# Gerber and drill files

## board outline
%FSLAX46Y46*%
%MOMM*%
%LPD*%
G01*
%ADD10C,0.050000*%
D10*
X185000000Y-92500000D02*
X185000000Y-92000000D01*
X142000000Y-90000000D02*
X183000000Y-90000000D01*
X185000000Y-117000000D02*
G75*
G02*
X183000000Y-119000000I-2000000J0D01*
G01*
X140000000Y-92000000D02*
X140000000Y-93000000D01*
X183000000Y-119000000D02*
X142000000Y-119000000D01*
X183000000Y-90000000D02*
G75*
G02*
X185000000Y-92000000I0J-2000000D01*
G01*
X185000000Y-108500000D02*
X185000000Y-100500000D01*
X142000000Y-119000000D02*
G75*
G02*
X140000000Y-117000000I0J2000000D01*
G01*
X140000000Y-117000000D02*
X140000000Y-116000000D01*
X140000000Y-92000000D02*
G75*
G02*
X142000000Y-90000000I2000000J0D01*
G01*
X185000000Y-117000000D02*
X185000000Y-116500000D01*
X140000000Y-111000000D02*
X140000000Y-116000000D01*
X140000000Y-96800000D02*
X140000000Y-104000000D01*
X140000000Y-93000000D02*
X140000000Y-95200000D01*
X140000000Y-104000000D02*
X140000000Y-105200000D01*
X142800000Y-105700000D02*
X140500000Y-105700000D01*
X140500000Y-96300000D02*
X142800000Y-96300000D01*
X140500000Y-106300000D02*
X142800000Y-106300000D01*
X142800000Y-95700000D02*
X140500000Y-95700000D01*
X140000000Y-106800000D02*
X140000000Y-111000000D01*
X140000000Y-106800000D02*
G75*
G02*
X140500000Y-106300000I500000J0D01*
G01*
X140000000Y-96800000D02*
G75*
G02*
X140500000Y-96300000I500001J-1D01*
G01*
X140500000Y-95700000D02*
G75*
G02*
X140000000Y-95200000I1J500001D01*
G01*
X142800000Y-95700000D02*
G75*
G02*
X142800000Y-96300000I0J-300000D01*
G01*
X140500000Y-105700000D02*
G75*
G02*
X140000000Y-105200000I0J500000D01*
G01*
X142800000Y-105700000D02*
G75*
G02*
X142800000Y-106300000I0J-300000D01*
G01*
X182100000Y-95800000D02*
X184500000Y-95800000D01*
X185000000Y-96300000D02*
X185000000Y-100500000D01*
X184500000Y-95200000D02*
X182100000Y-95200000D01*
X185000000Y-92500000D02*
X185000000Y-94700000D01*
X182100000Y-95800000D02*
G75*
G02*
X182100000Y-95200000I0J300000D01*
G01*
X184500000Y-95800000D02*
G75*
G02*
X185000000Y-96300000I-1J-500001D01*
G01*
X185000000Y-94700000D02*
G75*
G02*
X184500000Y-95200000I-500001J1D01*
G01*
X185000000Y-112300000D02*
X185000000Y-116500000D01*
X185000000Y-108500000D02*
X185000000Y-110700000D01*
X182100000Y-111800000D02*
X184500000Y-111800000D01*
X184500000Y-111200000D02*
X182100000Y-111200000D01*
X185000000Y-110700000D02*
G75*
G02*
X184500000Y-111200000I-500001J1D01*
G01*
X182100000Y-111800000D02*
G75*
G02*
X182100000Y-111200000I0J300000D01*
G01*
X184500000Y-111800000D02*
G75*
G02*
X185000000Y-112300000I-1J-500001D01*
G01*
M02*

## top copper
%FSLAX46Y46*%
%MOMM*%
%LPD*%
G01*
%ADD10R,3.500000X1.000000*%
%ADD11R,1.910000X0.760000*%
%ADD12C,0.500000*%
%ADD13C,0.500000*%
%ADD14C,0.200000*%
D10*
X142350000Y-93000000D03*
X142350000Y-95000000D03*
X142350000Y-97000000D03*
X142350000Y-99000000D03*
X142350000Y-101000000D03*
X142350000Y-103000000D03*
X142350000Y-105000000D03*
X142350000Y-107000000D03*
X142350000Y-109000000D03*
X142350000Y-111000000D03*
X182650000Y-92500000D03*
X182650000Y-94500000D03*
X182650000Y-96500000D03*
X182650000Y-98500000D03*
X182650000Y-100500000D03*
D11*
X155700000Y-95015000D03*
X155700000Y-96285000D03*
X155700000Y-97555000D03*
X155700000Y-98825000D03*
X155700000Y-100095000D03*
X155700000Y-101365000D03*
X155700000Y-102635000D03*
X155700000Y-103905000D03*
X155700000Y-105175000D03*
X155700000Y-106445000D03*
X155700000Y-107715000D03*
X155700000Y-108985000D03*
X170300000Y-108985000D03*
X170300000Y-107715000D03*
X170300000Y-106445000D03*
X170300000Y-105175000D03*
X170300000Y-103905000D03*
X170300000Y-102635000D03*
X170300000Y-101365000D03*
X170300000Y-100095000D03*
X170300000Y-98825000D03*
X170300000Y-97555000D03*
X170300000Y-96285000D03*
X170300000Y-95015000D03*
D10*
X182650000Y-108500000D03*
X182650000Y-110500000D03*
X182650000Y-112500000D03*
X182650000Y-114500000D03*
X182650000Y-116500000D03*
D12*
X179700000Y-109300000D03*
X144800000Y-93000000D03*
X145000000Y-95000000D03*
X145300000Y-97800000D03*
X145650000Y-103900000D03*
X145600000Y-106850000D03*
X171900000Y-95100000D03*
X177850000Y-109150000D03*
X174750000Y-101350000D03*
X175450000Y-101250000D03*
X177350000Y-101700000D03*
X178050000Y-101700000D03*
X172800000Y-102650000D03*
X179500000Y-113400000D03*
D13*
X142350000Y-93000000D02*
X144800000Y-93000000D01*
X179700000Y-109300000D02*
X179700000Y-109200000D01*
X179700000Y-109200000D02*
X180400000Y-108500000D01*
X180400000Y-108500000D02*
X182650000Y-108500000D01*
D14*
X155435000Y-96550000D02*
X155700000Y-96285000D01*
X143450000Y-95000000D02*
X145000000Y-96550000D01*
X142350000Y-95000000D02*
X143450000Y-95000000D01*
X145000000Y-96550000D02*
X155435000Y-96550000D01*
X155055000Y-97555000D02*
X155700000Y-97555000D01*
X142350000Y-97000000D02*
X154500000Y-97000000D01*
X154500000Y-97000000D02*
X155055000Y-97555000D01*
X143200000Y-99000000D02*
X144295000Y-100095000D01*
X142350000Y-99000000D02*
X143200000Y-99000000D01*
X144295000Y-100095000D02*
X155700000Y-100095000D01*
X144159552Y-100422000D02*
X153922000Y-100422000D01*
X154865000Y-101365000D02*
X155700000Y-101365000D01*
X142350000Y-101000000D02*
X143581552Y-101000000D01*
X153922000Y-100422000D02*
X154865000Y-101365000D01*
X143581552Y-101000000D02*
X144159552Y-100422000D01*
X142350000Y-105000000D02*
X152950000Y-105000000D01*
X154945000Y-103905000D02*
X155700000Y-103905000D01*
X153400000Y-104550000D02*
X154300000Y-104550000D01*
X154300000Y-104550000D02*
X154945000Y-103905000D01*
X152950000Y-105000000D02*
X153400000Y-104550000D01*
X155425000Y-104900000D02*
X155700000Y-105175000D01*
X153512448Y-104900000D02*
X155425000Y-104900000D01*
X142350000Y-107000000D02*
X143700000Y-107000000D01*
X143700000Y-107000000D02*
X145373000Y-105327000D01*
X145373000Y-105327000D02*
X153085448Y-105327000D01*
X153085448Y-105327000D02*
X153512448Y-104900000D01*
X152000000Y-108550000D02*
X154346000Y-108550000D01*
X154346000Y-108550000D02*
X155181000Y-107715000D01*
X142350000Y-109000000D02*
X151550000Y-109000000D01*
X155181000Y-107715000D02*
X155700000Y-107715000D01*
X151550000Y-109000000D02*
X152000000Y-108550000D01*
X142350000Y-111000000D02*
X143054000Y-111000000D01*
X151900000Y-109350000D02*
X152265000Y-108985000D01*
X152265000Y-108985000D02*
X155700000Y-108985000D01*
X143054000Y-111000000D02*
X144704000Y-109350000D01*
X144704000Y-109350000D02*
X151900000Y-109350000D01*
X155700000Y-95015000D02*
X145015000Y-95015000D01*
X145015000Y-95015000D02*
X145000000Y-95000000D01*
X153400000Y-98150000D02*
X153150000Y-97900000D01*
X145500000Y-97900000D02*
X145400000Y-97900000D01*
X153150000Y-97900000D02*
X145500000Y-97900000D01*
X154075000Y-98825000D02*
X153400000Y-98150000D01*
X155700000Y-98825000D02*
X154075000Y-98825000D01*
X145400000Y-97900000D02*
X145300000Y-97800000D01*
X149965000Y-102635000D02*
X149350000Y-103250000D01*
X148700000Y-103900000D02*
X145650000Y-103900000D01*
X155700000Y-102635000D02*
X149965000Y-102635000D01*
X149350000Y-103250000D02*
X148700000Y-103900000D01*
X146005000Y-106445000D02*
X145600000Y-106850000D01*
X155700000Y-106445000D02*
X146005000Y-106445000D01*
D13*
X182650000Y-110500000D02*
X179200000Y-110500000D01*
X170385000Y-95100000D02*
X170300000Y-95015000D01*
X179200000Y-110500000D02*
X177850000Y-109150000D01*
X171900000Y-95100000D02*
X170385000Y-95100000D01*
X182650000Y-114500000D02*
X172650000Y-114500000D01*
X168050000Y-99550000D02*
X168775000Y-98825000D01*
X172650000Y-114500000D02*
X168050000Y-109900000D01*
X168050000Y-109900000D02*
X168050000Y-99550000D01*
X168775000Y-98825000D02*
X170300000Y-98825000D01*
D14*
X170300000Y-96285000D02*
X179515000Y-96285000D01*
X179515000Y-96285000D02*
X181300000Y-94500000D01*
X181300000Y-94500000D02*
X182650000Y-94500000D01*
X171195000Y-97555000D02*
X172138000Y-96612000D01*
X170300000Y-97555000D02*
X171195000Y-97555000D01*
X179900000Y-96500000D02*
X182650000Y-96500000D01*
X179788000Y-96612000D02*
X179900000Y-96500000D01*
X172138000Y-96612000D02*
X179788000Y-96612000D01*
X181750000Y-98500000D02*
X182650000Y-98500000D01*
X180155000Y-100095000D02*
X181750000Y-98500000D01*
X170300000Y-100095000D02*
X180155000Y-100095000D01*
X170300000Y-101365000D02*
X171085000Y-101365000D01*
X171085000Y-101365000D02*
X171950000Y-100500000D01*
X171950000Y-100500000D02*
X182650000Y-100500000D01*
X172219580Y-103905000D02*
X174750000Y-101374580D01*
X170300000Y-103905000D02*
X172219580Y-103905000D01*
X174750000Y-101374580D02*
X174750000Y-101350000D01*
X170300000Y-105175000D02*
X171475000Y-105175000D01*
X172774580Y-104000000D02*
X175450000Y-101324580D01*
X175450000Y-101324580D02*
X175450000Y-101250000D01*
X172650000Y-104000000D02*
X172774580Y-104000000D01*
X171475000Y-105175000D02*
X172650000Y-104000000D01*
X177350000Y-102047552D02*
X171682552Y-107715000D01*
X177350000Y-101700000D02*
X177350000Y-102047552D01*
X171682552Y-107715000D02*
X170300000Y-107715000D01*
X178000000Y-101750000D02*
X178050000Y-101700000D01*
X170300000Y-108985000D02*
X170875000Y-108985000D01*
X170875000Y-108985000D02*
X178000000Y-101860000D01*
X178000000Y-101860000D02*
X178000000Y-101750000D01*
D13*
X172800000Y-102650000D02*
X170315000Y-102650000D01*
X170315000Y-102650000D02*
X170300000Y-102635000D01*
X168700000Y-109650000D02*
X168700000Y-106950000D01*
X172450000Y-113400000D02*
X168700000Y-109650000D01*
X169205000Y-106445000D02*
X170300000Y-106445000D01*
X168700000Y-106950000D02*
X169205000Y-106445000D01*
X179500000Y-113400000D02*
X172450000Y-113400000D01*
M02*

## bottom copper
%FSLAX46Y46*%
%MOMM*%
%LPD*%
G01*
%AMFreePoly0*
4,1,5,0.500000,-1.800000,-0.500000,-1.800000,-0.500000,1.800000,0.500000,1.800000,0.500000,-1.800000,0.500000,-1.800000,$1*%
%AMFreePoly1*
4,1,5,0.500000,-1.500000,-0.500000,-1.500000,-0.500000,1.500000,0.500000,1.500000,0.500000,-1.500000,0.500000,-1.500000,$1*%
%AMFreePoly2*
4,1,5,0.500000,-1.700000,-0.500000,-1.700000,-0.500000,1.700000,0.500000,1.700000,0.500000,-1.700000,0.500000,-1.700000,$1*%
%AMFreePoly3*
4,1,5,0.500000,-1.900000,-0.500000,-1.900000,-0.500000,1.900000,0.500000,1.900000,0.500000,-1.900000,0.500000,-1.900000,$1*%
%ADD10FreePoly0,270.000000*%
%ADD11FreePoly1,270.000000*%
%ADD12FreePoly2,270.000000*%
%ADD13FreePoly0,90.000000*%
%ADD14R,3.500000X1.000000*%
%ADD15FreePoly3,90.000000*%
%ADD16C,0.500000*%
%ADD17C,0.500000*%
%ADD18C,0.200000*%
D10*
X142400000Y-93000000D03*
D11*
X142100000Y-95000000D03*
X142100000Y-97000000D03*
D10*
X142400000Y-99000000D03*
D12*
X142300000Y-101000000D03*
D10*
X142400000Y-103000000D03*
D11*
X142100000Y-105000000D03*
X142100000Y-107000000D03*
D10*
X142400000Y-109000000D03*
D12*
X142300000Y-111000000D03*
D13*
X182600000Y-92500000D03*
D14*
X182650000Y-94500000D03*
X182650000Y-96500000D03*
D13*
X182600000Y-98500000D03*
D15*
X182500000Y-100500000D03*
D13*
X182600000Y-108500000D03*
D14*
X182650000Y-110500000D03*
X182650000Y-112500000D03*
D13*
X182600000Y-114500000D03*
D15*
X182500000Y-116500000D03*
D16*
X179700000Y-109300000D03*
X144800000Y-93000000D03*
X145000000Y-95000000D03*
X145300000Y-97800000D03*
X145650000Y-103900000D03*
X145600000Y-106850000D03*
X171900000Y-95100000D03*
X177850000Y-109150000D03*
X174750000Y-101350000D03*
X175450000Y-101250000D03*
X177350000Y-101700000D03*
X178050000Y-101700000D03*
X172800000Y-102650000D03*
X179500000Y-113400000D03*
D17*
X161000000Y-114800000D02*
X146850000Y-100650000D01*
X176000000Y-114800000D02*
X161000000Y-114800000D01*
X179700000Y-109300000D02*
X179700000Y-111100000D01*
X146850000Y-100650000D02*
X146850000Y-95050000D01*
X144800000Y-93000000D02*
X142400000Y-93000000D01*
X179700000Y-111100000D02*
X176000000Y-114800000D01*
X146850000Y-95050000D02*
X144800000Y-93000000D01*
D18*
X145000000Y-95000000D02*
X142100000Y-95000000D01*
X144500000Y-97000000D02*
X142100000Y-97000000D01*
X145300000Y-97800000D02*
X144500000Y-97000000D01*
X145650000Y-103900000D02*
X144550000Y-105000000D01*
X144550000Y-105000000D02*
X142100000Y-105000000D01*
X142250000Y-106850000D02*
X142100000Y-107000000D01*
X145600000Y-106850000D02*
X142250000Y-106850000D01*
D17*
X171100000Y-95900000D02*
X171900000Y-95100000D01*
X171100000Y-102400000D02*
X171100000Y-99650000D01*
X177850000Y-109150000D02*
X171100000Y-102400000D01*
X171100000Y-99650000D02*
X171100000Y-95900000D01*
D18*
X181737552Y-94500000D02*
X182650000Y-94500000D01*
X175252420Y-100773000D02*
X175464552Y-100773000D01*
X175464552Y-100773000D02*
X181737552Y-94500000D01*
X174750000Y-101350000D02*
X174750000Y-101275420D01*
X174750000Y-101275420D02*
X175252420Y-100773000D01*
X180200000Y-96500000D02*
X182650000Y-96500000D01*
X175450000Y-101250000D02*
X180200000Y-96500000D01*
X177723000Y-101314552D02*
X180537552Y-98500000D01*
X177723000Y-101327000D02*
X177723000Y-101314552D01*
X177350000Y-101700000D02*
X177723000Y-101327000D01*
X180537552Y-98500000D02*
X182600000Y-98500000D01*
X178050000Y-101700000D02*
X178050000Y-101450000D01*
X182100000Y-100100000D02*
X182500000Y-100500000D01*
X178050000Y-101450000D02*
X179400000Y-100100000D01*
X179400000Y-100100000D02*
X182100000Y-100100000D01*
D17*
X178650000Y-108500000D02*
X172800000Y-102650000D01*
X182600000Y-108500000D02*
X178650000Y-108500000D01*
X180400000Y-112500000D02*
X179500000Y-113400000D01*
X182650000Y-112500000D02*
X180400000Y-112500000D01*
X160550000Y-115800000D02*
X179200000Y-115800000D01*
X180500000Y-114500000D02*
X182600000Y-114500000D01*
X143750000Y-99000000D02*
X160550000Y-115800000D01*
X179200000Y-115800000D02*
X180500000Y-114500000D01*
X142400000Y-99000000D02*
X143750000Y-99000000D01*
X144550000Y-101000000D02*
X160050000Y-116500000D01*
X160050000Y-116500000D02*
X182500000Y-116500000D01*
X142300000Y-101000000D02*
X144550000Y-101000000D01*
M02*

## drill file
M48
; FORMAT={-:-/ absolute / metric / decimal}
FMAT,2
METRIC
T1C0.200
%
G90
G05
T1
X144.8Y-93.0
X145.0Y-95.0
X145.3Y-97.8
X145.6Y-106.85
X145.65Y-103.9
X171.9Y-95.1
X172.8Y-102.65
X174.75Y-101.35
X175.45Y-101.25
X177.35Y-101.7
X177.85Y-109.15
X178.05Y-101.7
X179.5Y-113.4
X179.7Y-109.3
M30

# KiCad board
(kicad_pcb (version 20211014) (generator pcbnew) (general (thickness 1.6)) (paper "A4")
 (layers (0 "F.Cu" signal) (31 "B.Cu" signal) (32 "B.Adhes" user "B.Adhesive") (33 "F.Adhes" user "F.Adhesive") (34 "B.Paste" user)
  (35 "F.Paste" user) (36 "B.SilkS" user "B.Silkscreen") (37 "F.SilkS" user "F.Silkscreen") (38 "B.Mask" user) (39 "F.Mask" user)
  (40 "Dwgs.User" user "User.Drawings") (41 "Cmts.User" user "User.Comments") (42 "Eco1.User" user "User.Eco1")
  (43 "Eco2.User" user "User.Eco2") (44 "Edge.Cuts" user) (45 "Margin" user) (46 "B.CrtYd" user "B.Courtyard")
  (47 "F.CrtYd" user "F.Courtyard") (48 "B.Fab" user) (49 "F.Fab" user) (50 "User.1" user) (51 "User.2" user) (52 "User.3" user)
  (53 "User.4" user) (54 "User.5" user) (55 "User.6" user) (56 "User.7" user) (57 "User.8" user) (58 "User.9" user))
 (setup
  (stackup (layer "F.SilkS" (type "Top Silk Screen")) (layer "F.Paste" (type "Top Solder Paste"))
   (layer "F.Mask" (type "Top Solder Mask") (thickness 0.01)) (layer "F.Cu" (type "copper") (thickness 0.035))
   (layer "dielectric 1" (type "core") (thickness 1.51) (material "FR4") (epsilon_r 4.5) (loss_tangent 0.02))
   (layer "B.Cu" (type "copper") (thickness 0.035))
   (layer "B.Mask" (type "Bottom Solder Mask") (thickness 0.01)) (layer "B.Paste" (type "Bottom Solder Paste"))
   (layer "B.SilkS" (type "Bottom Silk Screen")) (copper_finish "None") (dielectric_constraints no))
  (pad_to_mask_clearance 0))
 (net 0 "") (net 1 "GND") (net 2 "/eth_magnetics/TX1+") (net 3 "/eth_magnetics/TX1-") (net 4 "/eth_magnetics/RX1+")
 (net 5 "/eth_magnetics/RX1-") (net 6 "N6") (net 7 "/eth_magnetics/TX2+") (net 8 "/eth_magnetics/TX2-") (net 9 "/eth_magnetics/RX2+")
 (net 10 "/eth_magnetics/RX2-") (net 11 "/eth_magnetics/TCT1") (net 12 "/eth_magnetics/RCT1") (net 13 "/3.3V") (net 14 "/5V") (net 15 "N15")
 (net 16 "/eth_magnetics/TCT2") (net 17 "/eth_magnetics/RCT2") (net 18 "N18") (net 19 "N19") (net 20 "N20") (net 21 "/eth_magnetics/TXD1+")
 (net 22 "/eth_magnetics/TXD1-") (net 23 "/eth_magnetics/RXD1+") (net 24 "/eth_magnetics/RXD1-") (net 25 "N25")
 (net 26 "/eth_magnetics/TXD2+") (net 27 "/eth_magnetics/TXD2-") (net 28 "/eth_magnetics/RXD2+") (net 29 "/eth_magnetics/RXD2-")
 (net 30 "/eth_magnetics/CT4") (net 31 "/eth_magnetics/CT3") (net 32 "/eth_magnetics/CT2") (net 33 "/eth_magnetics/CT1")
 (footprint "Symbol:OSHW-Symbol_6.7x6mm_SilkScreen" (layer "F.Cu") (at 158 116)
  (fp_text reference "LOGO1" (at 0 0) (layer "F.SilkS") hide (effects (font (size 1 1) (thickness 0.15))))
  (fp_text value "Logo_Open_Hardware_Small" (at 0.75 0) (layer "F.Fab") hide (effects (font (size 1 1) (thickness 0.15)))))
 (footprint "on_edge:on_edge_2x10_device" (layer "F.Cu") (at 140 97 -90)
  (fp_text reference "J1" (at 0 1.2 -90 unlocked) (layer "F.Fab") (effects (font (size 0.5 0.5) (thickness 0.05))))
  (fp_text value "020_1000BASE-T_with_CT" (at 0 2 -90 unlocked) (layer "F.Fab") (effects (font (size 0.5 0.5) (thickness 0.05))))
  (fp_line (start -0.2 0) (end 7 0) (layer "Edge.Cuts") (width 0.05))
  (fp_line (start -4 0) (end -1.8 0) (layer "Edge.Cuts") (width 0.05))
  (fp_line (start 7 0) (end 8.2 0) (layer "Edge.Cuts") (width 0.05))
  (fp_line (start 8.7 -2.8) (end 8.7 -0.5) (layer "Edge.Cuts") (width 0.05))
  (fp_line (start -0.7 -0.5) (end -0.7 -2.8) (layer "Edge.Cuts") (width 0.05))
  (fp_line (start 9.3 -0.5) (end 9.3 -2.8) (layer "Edge.Cuts") (width 0.05))
  (fp_line (start -1.3 -2.8) (end -1.3 -0.5) (layer "Edge.Cuts") (width 0.05))
  (fp_line (start 9.8 0) (end 14 0) (layer "Edge.Cuts") (width 0.05))
  (fp_arc (start 9.8 0) (mid 9.446447 -0.146447) (end 9.3 -0.5) (layer "Edge.Cuts") (width 0.05))
  (fp_arc (start -0.2 0) (mid -0.553553 -0.146447) (end -0.7 -0.5) (layer "Edge.Cuts") (width 0.05))
  (fp_arc (start -1.3 -0.5) (mid -1.446447 -0.146447) (end -1.8 0) (layer "Edge.Cuts") (width 0.05))
  (fp_arc (start -1.3 -2.8) (mid -1 -3.1) (end -0.7 -2.8) (layer "Edge.Cuts") (width 0.05))
  (fp_arc (start 8.7 -0.5) (mid 8.553553 -0.146447) (end 8.2 0) (layer "Edge.Cuts") (width 0.05))
  (fp_arc (start 8.7 -2.8) (mid 9 -3.1) (end 9.3 -2.8) (layer "Edge.Cuts") (width 0.05))
  (pad "1" smd rect (at -4 -2.35 90) (size 1 3.5) (layers "F.Cu" "F.Mask") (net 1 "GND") (zone_connect 0))
  (pad "2" smd rect (at -2 -2.35 270) (size 1 3.5) (layers "F.Cu" "F.Mask") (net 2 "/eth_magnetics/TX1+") (zone_connect 0))
  (pad "3" smd rect (at 0 -2.35 270) (size 1 3.5) (layers "F.Cu" "F.Mask") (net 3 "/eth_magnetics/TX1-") (zone_connect 0))
  (pad "4" smd rect (at 2 -2.35 90) (size 1 3.5) (layers "F.Cu" "F.Mask") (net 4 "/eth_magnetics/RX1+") (zone_connect 0))
  (pad "5" smd rect (at 4 -2.35 90) (size 1 3.5) (layers "F.Cu" "F.Mask") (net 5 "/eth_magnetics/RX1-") (zone_connect 0))
  (pad "6" smd rect (at 6 -2.35 90) (size 1 3.5) (layers "F.Cu" "F.Mask") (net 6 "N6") (zone_connect 0))
  (pad "7" smd rect (at 8 -2.35 270) (size 1 3.5) (layers "F.Cu" "F.Mask") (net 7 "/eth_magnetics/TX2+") (zone_connect 0))
  (pad "8" smd rect (at 10 -2.35 270) (size 1 3.5) (layers "F.Cu" "F.Mask") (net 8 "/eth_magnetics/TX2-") (zone_connect 0))
  (pad "9" smd rect (at 12 -2.35 90) (size 1 3.5) (layers "F.Cu" "F.Mask") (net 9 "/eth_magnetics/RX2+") (zone_connect 0))
  (pad "10" smd rect (at 14 -2.35 90) (size 1 3.5) (layers "F.Cu" "F.Mask") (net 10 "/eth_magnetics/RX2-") (zone_connect 0))
  (pad "11" smd custom (at -4 -2.4 270) (size 1 3.6) (layers "B.Cu" "B.Mask") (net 1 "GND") (zone_connect 0)
   (options (clearance outline) (anchor rect)) (primitives))
  (pad "12" smd custom (at -2 -2.1 270) (size 1 3) (layers "B.Cu" "B.Mask") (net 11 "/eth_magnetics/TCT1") (zone_connect 0)
   (options (clearance outline) (anchor rect)) (primitives))
  (pad "13" smd custom (at 0 -2.1 270) (size 1 3) (layers "B.Cu" "B.Mask") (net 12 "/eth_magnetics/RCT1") (zone_connect 0)
   (options (clearance outline) (anchor rect)) (primitives))
  (pad "14" smd custom (at 2 -2.4 270) (size 1 3.6) (layers "B.Cu" "B.Mask") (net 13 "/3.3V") (zone_connect 0)
   (options (clearance outline) (anchor rect)) (primitives))
  (pad "15" smd custom (at 4 -2.3 270) (size 1 3.4) (layers "B.Cu" "B.Mask") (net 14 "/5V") (zone_connect 0)
   (options (clearance outline) (anchor rect)) (primitives))
  (pad "16" smd custom (at 6 -2.4 270) (size 1 3.6) (layers "B.Cu" "B.Mask") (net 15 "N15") (zone_connect 0)
   (options (clearance outline) (anchor rect)) (primitives))
  (pad "17" smd custom (at 8 -2.1 270) (size 1 3) (layers "B.Cu" "B.Mask") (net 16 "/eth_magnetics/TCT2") (zone_connect 0)
   (options (clearance outline) (anchor rect)) (primitives))
  (pad "18" smd custom (at 10 -2.1 270) (size 1 3) (layers "B.Cu" "B.Mask") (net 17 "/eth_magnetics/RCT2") (zone_connect 0)
   (options (clearance outline) (anchor rect)) (primitives))
  (pad "19" smd custom (at 12 -2.4 270) (size 1 3.6) (layers "B.Cu" "B.Mask") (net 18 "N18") (zone_connect 0)
   (options (clearance outline) (anchor rect)) (primitives))
  (pad "20" smd custom (at 14 -2.3 270) (size 1 3.4) (layers "B.Cu" "B.Mask") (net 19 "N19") (zone_connect 0)
   (options (clearance outline) (anchor rect)) (primitives))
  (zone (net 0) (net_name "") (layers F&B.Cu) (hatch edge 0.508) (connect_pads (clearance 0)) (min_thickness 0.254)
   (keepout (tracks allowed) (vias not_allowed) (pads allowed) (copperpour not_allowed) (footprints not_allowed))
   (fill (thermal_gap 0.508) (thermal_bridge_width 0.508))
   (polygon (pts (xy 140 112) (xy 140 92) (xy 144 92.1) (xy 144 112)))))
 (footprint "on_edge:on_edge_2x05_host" (layer "F.Cu") (at 185 96.5 -90)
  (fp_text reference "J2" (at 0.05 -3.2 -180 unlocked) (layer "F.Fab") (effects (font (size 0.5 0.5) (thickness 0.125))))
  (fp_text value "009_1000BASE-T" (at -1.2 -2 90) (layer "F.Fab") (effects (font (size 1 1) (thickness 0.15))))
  (fp_line (start -0.7 2.9) (end -0.7 0.5) (layer "Edge.Cuts") (width 0.05))
  (fp_line (start -0.2 0) (end 4 0) (layer "Edge.Cuts") (width 0.05))
  (fp_line (start -1.3 0.5) (end -1.3 2.9) (layer "Edge.Cuts") (width 0.05))
  (fp_line (start -4 0) (end -1.8 0) (layer "Edge.Cuts") (width 0.05))
  (fp_arc (start -0.7 2.9) (mid -1 3.2) (end -1.3 2.9) (layer "Edge.Cuts") (width 0.05))
  (fp_arc (start -0.7 0.5) (mid -0.553553 0.146447) (end -0.2 0) (layer "Edge.Cuts") (width 0.05))
  (fp_arc (start -1.8 0) (mid -1.446447 0.146447) (end -1.3 0.5) (layer "Edge.Cuts") (width 0.05))
  (pad "1" smd rect (at -4 2.35 270) (size 1 3.5) (layers "F.Cu" "F.Mask") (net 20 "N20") (zone_connect 0))
  (pad "2" smd rect (at -2 2.35 270) (size 1 3.5) (layers "F.Cu" "F.Mask") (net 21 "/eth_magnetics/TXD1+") (zone_connect 0))
  (pad "3" smd rect (at 0 2.35 270) (size 1 3.5) (layers "F.Cu" "F.Mask") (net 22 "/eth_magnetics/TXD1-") (zone_connect 0))
  (pad "4" smd rect (at 2 2.35 270) (size 1 3.5) (layers "F.Cu" "F.Mask") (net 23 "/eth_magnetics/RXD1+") (zone_connect 0))
  (pad "5" smd rect (at 4 2.35 270) (size 1 3.5) (layers "F.Cu" "F.Mask") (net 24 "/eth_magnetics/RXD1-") (zone_connect 0))
  (pad "6" smd custom (at -4 2.4 90) (size 1 3.6) (layers "B.Cu" "B.Mask") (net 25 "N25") (zone_connect 0)
   (options (clearance outline) (anchor rect)) (primitives))
  (pad "7" smd rect (at -2 2.35 90) (size 1 3.5) (layers "B.Cu" "B.Mask") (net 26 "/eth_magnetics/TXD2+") (zone_connect 0))
  (pad "8" smd rect (at 0 2.35 90) (size 1 3.5) (layers "B.Cu" "B.Mask") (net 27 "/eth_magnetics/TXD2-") (zone_connect 0))
  (pad "9" smd custom (at 2 2.4 90) (size 1 3.6) (layers "B.Cu" "B.Mask") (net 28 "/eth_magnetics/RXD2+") (zone_connect 0)
   (options (clearance outline) (anchor rect)) (primitives))
  (pad "10" smd custom (at 4 2.5 90) (size 1 3.8) (layers "B.Cu" "B.Mask") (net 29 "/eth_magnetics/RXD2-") (zone_connect 0)
   (options (clearance outline) (anchor rect)) (primitives))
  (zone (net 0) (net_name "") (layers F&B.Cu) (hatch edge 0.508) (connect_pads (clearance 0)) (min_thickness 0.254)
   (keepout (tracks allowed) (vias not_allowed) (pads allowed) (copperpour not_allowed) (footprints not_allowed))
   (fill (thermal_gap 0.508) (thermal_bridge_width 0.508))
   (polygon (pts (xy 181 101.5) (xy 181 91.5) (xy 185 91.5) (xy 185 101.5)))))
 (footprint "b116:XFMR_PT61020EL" (layer "F.Cu") (at 163 102)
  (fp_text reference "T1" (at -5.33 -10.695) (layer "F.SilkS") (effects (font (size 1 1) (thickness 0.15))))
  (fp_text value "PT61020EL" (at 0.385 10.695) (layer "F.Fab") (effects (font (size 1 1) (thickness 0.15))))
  (pad "1" smd rect (at -7.3 -6.985) (size 1.91 0.76) (layers "F.Cu" "F.Paste" "F.Mask") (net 11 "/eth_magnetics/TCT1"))
  (pad "2" smd rect (at -7.3 -5.715) (size 1.91 0.76) (layers "F.Cu" "F.Paste" "F.Mask") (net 2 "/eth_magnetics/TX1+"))
  (pad "3" smd rect (at -7.3 -4.445) (size 1.91 0.76) (layers "F.Cu" "F.Paste" "F.Mask") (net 3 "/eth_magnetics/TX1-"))
  (pad "4" smd rect (at -7.3 -3.175) (size 1.91 0.76) (layers "F.Cu" "F.Paste" "F.Mask") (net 12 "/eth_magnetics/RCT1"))
  (pad "5" smd rect (at -7.3 -1.905) (size 1.91 0.76) (layers "F.Cu" "F.Paste" "F.Mask") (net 4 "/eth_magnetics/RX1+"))
  (pad "6" smd rect (at -7.3 -0.635) (size 1.91 0.76) (layers "F.Cu" "F.Paste" "F.Mask") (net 5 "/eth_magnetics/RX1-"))
  (pad "7" smd rect (at -7.3 0.635) (size 1.91 0.76) (layers "F.Cu" "F.Paste" "F.Mask") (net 16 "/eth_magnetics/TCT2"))
  (pad "8" smd rect (at -7.3 1.905) (size 1.91 0.76) (layers "F.Cu" "F.Paste" "F.Mask") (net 7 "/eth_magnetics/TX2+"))
  (pad "9" smd rect (at -7.3 3.175) (size 1.91 0.76) (layers "F.Cu" "F.Paste" "F.Mask") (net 8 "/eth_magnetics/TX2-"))
  (pad "10" smd rect (at -7.3 4.445) (size 1.91 0.76) (layers "F.Cu" "F.Paste" "F.Mask") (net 17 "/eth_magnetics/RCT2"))
  (pad "11" smd rect (at -7.3 5.715) (size 1.91 0.76) (layers "F.Cu" "F.Paste" "F.Mask") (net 9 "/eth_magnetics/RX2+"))
  (pad "12" smd rect (at -7.3 6.985) (size 1.91 0.76) (layers "F.Cu" "F.Paste" "F.Mask") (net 10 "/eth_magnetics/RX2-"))
  (pad "13" smd rect (at 7.3 6.985) (size 1.91 0.76) (layers "F.Cu" "F.Paste" "F.Mask") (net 29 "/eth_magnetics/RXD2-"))
  (pad "14" smd rect (at 7.3 5.715) (size 1.91 0.76) (layers "F.Cu" "F.Paste" "F.Mask") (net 28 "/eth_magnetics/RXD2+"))
  (pad "15" smd rect (at 7.3 4.445) (size 1.91 0.76) (layers "F.Cu" "F.Paste" "F.Mask") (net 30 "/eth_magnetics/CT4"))
  (pad "16" smd rect (at 7.3 3.175) (size 1.91 0.76) (layers "F.Cu" "F.Paste" "F.Mask") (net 27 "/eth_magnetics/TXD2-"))
  (pad "17" smd rect (at 7.3 1.905) (size 1.91 0.76) (layers "F.Cu" "F.Paste" "F.Mask") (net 26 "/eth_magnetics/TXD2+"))
  (pad "18" smd rect (at 7.3 0.635) (size 1.91 0.76) (layers "F.Cu" "F.Paste" "F.Mask") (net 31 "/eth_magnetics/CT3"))
  (pad "19" smd rect (at 7.3 -0.635) (size 1.91 0.76) (layers "F.Cu" "F.Paste" "F.Mask") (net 24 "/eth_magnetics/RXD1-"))
  (pad "20" smd rect (at 7.3 -1.905) (size 1.91 0.76) (layers "F.Cu" "F.Paste" "F.Mask") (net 23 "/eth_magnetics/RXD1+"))
  (pad "21" smd rect (at 7.3 -3.175) (size 1.91 0.76) (layers "F.Cu" "F.Paste" "F.Mask") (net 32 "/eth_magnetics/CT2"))
  (pad "22" smd rect (at 7.3 -4.445) (size 1.91 0.76) (layers "F.Cu" "F.Paste" "F.Mask") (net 22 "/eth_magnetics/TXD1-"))
  (pad "23" smd rect (at 7.3 -5.715) (size 1.91 0.76) (layers "F.Cu" "F.Paste" "F.Mask") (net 21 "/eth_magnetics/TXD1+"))
  (pad "24" smd rect (at 7.3 -6.985) (size 1.91 0.76) (layers "F.Cu" "F.Paste" "F.Mask") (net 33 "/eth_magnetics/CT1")))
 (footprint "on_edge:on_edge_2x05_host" (layer "F.Cu") (at 185 112.5 -90)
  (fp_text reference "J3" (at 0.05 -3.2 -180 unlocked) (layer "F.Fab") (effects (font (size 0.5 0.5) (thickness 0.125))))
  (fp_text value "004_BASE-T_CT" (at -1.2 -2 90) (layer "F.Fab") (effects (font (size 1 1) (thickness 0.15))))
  (fp_line (start -0.2 0) (end 4 0) (layer "Edge.Cuts") (width 0.05))
  (fp_line (start -4 0) (end -1.8 0) (layer "Edge.Cuts") (width 0.05))
  (fp_line (start -0.7 2.9) (end -0.7 0.5) (layer "Edge.Cuts") (width 0.05))
  (fp_line (start -1.3 0.5) (end -1.3 2.9) (layer "Edge.Cuts") (width 0.05))
  (fp_arc (start -1.8 0) (mid -1.446447 0.146447) (end -1.3 0.5) (layer "Edge.Cuts") (width 0.05))
  (fp_arc (start -0.7 2.9) (mid -1 3.2) (end -1.3 2.9) (layer "Edge.Cuts") (width 0.05))
  (fp_arc (start -0.7 0.5) (mid -0.553553 0.146447) (end -0.2 0) (layer "Edge.Cuts") (width 0.05))
  (pad "1" smd rect (at -4 2.35 270) (size 1 3.5) (layers "F.Cu" "F.Mask") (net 1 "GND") (zone_connect 0))
  (pad "2" smd rect (at -2 2.35 270) (size 1 3.5) (layers "F.Cu" "F.Mask") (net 33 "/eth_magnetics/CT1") (zone_connect 0))
  (pad "3" smd rect (at 0 2.35 270) (size 1 3.5) (layers "F.Cu" "F.Mask") (zone_connect 0))
  (pad "4" smd rect (at 2 2.35 270) (size 1 3.5) (layers "F.Cu" "F.Mask") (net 32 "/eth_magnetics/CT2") (zone_connect 0))
  (pad "5" smd rect (at 4 2.35 270) (size 1 3.5) (layers "F.Cu" "F.Mask") (zone_connect 0))
  (pad "6" smd custom (at -4 2.4 90) (size 1 3.6) (layers "B.Cu" "B.Mask") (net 31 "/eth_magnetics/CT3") (zone_connect 0)
   (options (clearance outline) (anchor rect)) (primitives))
  (pad "7" smd rect (at -2 2.35 90) (size 1 3.5) (layers "B.Cu" "B.Mask") (zone_connect 0))
  (pad "8" smd rect (at 0 2.35 90) (size 1 3.5) (layers "B.Cu" "B.Mask") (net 30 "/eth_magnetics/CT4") (zone_connect 0))
  (pad "9" smd custom (at 2 2.4 90) (size 1 3.6) (layers "B.Cu" "B.Mask") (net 13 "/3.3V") (zone_connect 0)
   (options (clearance outline) (anchor rect)) (primitives))
  (pad "10" smd custom (at 4 2.5 90) (size 1 3.8) (layers "B.Cu" "B.Mask") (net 14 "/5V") (zone_connect 0)
   (options (clearance outline) (anchor rect)) (primitives))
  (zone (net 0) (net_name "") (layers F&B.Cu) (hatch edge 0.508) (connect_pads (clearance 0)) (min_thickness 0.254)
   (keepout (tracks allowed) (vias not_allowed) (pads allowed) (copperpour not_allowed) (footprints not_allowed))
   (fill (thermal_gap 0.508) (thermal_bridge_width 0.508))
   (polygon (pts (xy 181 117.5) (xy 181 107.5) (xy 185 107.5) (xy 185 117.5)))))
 (gr_line (start 185 92.5) (end 185 92) (layer "Edge.Cuts") (width 0.05))
 (gr_line (start 142 90) (end 183 90) (layer "Edge.Cuts") (width 0.05))
 (gr_arc (start 185 117) (mid 184.414214 118.414214) (end 183 119) (layer "Edge.Cuts") (width 0.05))
 (gr_line (start 140 92) (end 140 93) (layer "Edge.Cuts") (width 0.05))
 (gr_line (start 183 119) (end 142 119) (layer "Edge.Cuts") (width 0.05))
 (gr_arc (start 183 90) (mid 184.414214 90.585786) (end 185 92) (layer "Edge.Cuts") (width 0.05))
 (gr_line (start 185 108.5) (end 185 100.5) (layer "Edge.Cuts") (width 0.05))
 (gr_arc (start 142 119) (mid 140.585786 118.414214) (end 140 117) (layer "Edge.Cuts") (width 0.05))
 (gr_line (start 140 117) (end 140 116) (layer "Edge.Cuts") (width 0.05))
 (gr_arc (start 140 92) (mid 140.585786 90.585786) (end 142 90) (layer "Edge.Cuts") (width 0.05))
 (gr_line (start 185 117) (end 185 116.5) (layer "Edge.Cuts") (width 0.05))
 (gr_line (start 140 111) (end 140 116) (layer "Edge.Cuts") (width 0.05))
 (segment (start 142.35 93) (end 144.8 93) (width 0.5) (layer "F.Cu") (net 1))
 (segment (start 179.7 109.3) (end 179.7 109.2) (width 0.5) (layer "F.Cu") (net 1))
 (segment (start 179.7 109.2) (end 180.4 108.5) (width 0.5) (layer "F.Cu") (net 1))
 (segment (start 180.4 108.5) (end 182.65 108.5) (width 0.5) (layer "F.Cu") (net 1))
 (via (at 179.7 109.3) (size 0.5) (drill 0.2) (layers "F.Cu" "B.Cu") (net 1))
 (via (at 144.8 93) (size 0.5) (drill 0.2) (layers "F.Cu" "B.Cu") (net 1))
 (segment (start 161 114.8) (end 146.85 100.65) (width 0.5) (layer "B.Cu") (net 1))
 (segment (start 176 114.8) (end 161 114.8) (width 0.5) (layer "B.Cu") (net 1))
 (segment (start 179.7 109.3) (end 179.7 111.1) (width 0.5) (layer "B.Cu") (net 1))
 (segment (start 146.85 100.65) (end 146.85 95.05) (width 0.5) (layer "B.Cu") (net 1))
 (segment (start 144.8 93) (end 142.4 93) (width 0.5) (layer "B.Cu") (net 1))
 (segment (start 179.7 111.1) (end 176 114.8) (width 0.5) (layer "B.Cu") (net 1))
 (segment (start 146.85 95.05) (end 144.8 93) (width 0.5) (layer "B.Cu") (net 1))
 (segment (start 155.435 96.55) (end 155.7 96.285) (width 0.2) (layer "F.Cu") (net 2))
 (segment (start 143.45 95) (end 145 96.55) (width 0.2) (layer "F.Cu") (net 2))
 (segment (start 142.35 95) (end 143.45 95) (width 0.2) (layer "F.Cu") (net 2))
 (segment (start 145 96.55) (end 155.435 96.55) (width 0.2) (layer "F.Cu") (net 2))
 (segment (start 155.055 97.555) (end 155.7 97.555) (width 0.2) (layer "F.Cu") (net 3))
 (segment (start 142.35 97) (end 154.5 97) (width 0.2) (layer "F.Cu") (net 3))
 (segment (start 154.5 97) (end 155.055 97.555) (width 0.2) (layer "F.Cu") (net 3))
 (segment (start 143.2 99) (end 144.295 100.095) (width 0.2) (layer "F.Cu") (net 4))
 (segment (start 142.35 99) (end 143.2 99) (width 0.2) (layer "F.Cu") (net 4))
 (segment (start 144.295 100.095) (end 155.7 100.095) (width 0.2) (layer "F.Cu") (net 4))
 (segment (start 144.159552 100.422) (end 153.922 100.422) (width 0.2) (layer "F.Cu") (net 5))
 (segment (start 154.865 101.365) (end 155.7 101.365) (width 0.2) (layer "F.Cu") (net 5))
 (segment (start 142.35 101) (end 143.581552 101) (width 0.2) (layer "F.Cu") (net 5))
 (segment (start 153.922 100.422) (end 154.865 101.365) (width 0.2) (layer "F.Cu") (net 5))
 (segment (start 143.581552 101) (end 144.159552 100.422) (width 0.2) (layer "F.Cu") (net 5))
 (segment (start 142.35 105) (end 152.95 105) (width 0.2) (layer "F.Cu") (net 7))
 (segment (start 154.945 103.905) (end 155.7 103.905) (width 0.2) (layer "F.Cu") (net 7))
 (segment (start 153.4 104.55) (end 154.3 104.55) (width 0.2) (layer "F.Cu") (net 7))
 (segment (start 154.3 104.55) (end 154.945 103.905) (width 0.2) (layer "F.Cu") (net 7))
 (segment (start 152.95 105) (end 153.4 104.55) (width 0.2) (layer "F.Cu") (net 7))
 (segment (start 155.425 104.9) (end 155.7 105.175) (width 0.2) (layer "F.Cu") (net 8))
 (segment (start 153.512448 104.9) (end 155.425 104.9) (width 0.2) (layer "F.Cu") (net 8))
 (segment (start 142.35 107) (end 143.7 107) (width 0.2) (layer "F.Cu") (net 8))
 (segment (start 143.7 107) (end 145.373 105.327) (width 0.2) (layer "F.Cu") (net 8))
 (segment (start 145.373 105.327) (end 153.085448 105.327) (width 0.2) (layer "F.Cu") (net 8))
 (segment (start 153.085448 105.327) (end 153.512448 104.9) (width 0.2) (layer "F.Cu") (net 8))
 (segment (start 152 108.55) (end 154.346 108.55) (width 0.2) (layer "F.Cu") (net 9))
 (segment (start 154.346 108.55) (end 155.181 107.715) (width 0.2) (layer "F.Cu") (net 9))
 (segment (start 142.35 109) (end 151.55 109) (width 0.2) (layer "F.Cu") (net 9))
 (segment (start 155.181 107.715) (end 155.7 107.715) (width 0.2) (layer "F.Cu") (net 9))
 (segment (start 151.55 109) (end 152 108.55) (width 0.2) (layer "F.Cu") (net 9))
 (segment (start 142.35 111) (end 143.054 111) (width 0.2) (layer "F.Cu") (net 10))
 (segment (start 151.9 109.35) (end 152.265 108.985) (width 0.2) (layer "F.Cu") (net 10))
 (segment (start 152.265 108.985) (end 155.7 108.985) (width 0.2) (layer "F.Cu") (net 10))
 (segment (start 143.054 111) (end 144.704 109.35) (width 0.2) (layer "F.Cu") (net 10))
 (segment (start 144.704 109.35) (end 151.9 109.35) (width 0.2) (layer "F.Cu") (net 10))
 (segment (start 155.7 95.015) (end 145.015 95.015) (width 0.2) (layer "F.Cu") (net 11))
 (segment (start 145.015 95.015) (end 145 95) (width 0.2) (layer "F.Cu") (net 11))
 (via (at 145 95) (size 0.5) (drill 0.2) (layers "F.Cu" "B.Cu") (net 11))
 (segment (start 145 95) (end 142.1 95) (width 0.2) (layer "B.Cu") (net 11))
 (segment (start 153.4 98.15) (end 153.15 97.9) (width 0.2) (layer "F.Cu") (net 12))
 (segment (start 145.5 97.9) (end 145.4 97.9) (width 0.2) (layer "F.Cu") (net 12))
 (segment (start 153.15 97.9) (end 145.5 97.9) (width 0.2) (layer "F.Cu") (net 12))
 (segment (start 154.075 98.825) (end 153.4 98.15) (width 0.2) (layer "F.Cu") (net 12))
 (segment (start 155.7 98.825) (end 154.075 98.825) (width 0.2) (layer "F.Cu") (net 12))
 (segment (start 145.4 97.9) (end 145.3 97.8) (width 0.2) (layer "F.Cu") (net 12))
 (via (at 145.3 97.8) (size 0.5) (drill 0.2) (layers "F.Cu" "B.Cu") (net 12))
 (segment (start 144.5 97) (end 142.1 97) (width 0.2) (layer "B.Cu") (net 12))
 (segment (start 145.3 97.8) (end 144.5 97) (width 0.2) (layer "B.Cu") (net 12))
 (segment (start 149.965 102.635) (end 149.35 103.25) (width 0.2) (layer "F.Cu") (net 16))
 (segment (start 148.7 103.9) (end 145.65 103.9) (width 0.2) (layer "F.Cu") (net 16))
 (segment (start 155.7 102.635) (end 149.965 102.635) (width 0.2) (layer "F.Cu") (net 16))
 (segment (start 149.35 103.25) (end 148.7 103.9) (width 0.2) (layer "F.Cu") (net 16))
 (via (at 145.65 103.9) (size 0.5) (drill 0.2) (layers "F.Cu" "B.Cu") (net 16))
 (segment (start 145.65 103.9) (end 144.55 105) (width 0.2) (layer "B.Cu") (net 16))
 (segment (start 144.55 105) (end 142.1 105) (width 0.2) (layer "B.Cu") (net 16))
 (segment (start 146.005 106.445) (end 145.6 106.85) (width 0.2) (layer "F.Cu") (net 17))
 (segment (start 155.7 106.445) (end 146.005 106.445) (width 0.2) (layer "F.Cu") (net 17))
 (via (at 145.6 106.85) (size 0.5) (drill 0.2) (layers "F.Cu" "B.Cu") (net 17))
 (segment (start 142.25 106.85) (end 142.1 107) (width 0.2) (layer "B.Cu") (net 17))
 (segment (start 145.6 106.85) (end 142.25 106.85) (width 0.2) (layer "B.Cu") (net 17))
 (segment (start 182.65 110.5) (end 179.2 110.5) (width 0.5) (layer "F.Cu") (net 33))
 (segment (start 170.385 95.1) (end 170.3 95.015) (width 0.5) (layer "F.Cu") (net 33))
 (segment (start 179.2 110.5) (end 177.85 109.15) (width 0.5) (layer "F.Cu") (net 33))
 (segment (start 171.9 95.1) (end 170.385 95.1) (width 0.5) (layer "F.Cu") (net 33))
 (via (at 171.9 95.1) (size 0.5) (drill 0.2) (layers "F.Cu" "B.Cu") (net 33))
 (via (at 177.85 109.15) (size 0.5) (drill 0.2) (layers "F.Cu" "B.Cu") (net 33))
 (segment (start 171.1 95.9) (end 171.9 95.1) (width 0.5) (layer "B.Cu") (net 33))
 (segment (start 171.1 102.4) (end 171.1 99.65) (width 0.5) (layer "B.Cu") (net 33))
 (segment (start 177.85 109.15) (end 171.1 102.4) (width 0.5) (layer "B.Cu") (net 33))
 (segment (start 171.1 99.65) (end 171.1 95.9) (width 0.5) (layer "B.Cu") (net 33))
 (segment (start 182.65 114.5) (end 172.65 114.5) (width 0.5) (layer "F.Cu") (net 32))
 (segment (start 168.05 99.55) (end 168.775 98.825) (width 0.5) (layer "F.Cu") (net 32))
 (segment (start 172.65 114.5) (end 168.05 109.9) (width 0.5) (layer "F.Cu") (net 32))
 (segment (start 168.05 109.9) (end 168.05 99.55) (width 0.5) (layer "F.Cu") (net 32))
 (segment (start 168.775 98.825) (end 170.3 98.825) (width 0.5) (layer "F.Cu") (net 32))
 (segment (start 170.3 96.285) (end 179.515 96.285) (width 0.2) (layer "F.Cu") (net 21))
 (segment (start 179.515 96.285) (end 181.3 94.5) (width 0.2) (layer "F.Cu") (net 21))
 (segment (start 181.3 94.5) (end 182.65 94.5) (width 0.2) (layer "F.Cu") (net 21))
 (segment (start 171.195 97.555) (end 172.138 96.612) (width 0.2) (layer "F.Cu") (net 22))
 (segment (start 170.3 97.555) (end 171.195 97.555) (width 0.2) (layer "F.Cu") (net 22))
 (segment (start 179.9 96.5) (end 182.65 96.5) (width 0.2) (layer "F.Cu") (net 22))
 (segment (start 179.788 96.612) (end 179.9 96.5) (width 0.2) (layer "F.Cu") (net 22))
 (segment (start 172.138 96.612) (end 179.788 96.612) (width 0.2) (layer "F.Cu") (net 22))
 (segment (start 181.75 98.5) (end 182.65 98.5) (width 0.2) (layer "F.Cu") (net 23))
 (segment (start 180.155 100.095) (end 181.75 98.5) (width 0.2) (layer "F.Cu") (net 23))
 (segment (start 170.3 100.095) (end 180.155 100.095) (width 0.2) (layer "F.Cu") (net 23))
 (segment (start 170.3 101.365) (end 171.085 101.365) (width 0.2) (layer "F.Cu") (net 24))
 (segment (start 171.085 101.365) (end 171.95 100.5) (width 0.2) (layer "F.Cu") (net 24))
 (segment (start 171.95 100.5) (end 182.65 100.5) (width 0.2) (layer "F.Cu") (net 24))
 (segment (start 172.21958 103.905) (end 174.75 101.37458) (width 0.2) (layer "F.Cu") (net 26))
 (segment (start 170.3 103.905) (end 172.21958 103.905) (width 0.2) (layer "F.Cu") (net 26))
 (segment (start 174.75 101.37458) (end 174.75 101.35) (width 0.2) (layer "F.Cu") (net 26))
 (via (at 174.75 101.35) (size 0.5) (drill 0.2) (layers "F.Cu" "B.Cu") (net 26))
 (segment (start 181.737552 94.5) (end 182.65 94.5) (width 0.2) (layer "B.Cu") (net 26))
 (segment (start 175.25242 100.773) (end 175.464552 100.773) (width 0.2) (layer "B.Cu") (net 26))
 (segment (start 175.464552 100.773) (end 181.737552 94.5) (width 0.2) (layer "B.Cu") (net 26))
 (segment (start 174.75 101.35) (end 174.75 101.27542) (width 0.2) (layer "B.Cu") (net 26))
 (segment (start 174.75 101.27542) (end 175.25242 100.773) (width 0.2) (layer "B.Cu") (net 26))
 (segment (start 170.3 105.175) (end 171.475 105.175) (width 0.2) (layer "F.Cu") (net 27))
 (segment (start 172.77458 104) (end 175.45 101.32458) (width 0.2) (layer "F.Cu") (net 27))
 (segment (start 175.45 101.32458) (end 175.45 101.25) (width 0.2) (layer "F.Cu") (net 27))
 (segment (start 172.65 104) (end 172.77458 104) (width 0.2) (layer "F.Cu") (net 27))
 (segment (start 171.475 105.175) (end 172.65 104) (width 0.2) (layer "F.Cu") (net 27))
 (via (at 175.45 101.25) (size 0.5) (drill 0.2) (layers "F.Cu" "B.Cu") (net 27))
 (segment (start 180.2 96.5) (end 182.65 96.5) (width 0.2) (layer "B.Cu") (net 27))
 (segment (start 175.45 101.25) (end 180.2 96.5) (width 0.2) (layer "B.Cu") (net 27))
 (segment (start 177.35 102.047552) (end 171.682552 107.715) (width 0.2) (layer "F.Cu") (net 28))
 (segment (start 177.35 101.7) (end 177.35 102.047552) (width 0.2) (layer "F.Cu") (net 28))
 (segment (start 171.682552 107.715) (end 170.3 107.715) (width 0.2) (layer "F.Cu") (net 28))
 (via (at 177.35 101.7) (size 0.5) (drill 0.2) (layers "F.Cu" "B.Cu") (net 28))
 (segment (start 177.723 101.314552) (end 180.537552 98.5) (width 0.2) (layer "B.Cu") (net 28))
 (segment (start 177.723 101.327) (end 177.723 101.314552) (width 0.2) (layer "B.Cu") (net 28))
 (segment (start 177.35 101.7) (end 177.723 101.327) (width 0.2) (layer "B.Cu") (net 28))
 (segment (start 180.537552 98.5) (end 182.6 98.5) (width 0.2) (layer "B.Cu") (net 28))
 (segment (start 178 101.75) (end 178.05 101.7) (width 0.2) (layer "F.Cu") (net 29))
 (segment (start 170.3 108.985) (end 170.875 108.985) (width 0.2) (layer "F.Cu") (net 29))
 (segment (start 170.875 108.985) (end 178 101.86) (width 0.2) (layer "F.Cu") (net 29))
 (segment (start 178 101.86) (end 178 101.75) (width 0.2) (layer "F.Cu") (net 29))
 (via (at 178.05 101.7) (size 0.5) (drill 0.2) (layers "F.Cu" "B.Cu") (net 29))
 (segment (start 178.05 101.7) (end 178.05 101.45) (width 0.2) (layer "B.Cu") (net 29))
 (segment (start 182.1 100.1) (end 182.5 100.5) (width 0.2) (layer "B.Cu") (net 29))
 (segment (start 178.05 101.45) (end 179.4 100.1) (width 0.2) (layer "B.Cu") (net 29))
 (segment (start 179.4 100.1) (end 182.1 100.1) (width 0.2) (layer "B.Cu") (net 29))
 (segment (start 172.8 102.65) (end 170.315 102.65) (width 0.5) (layer "F.Cu") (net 31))
 (segment (start 170.315 102.65) (end 170.3 102.635) (width 0.5) (layer "F.Cu") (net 31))
 (via (at 172.8 102.65) (size 0.5) (drill 0.2) (layers "F.Cu" "B.Cu") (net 31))
 (segment (start 178.65 108.5) (end 172.8 102.65) (width 0.5) (layer "B.Cu") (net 31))
 (segment (start 182.6 108.5) (end 178.65 108.5) (width 0.5) (layer "B.Cu") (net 31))
 (segment (start 168.7 109.65) (end 168.7 106.95) (width 0.5) (layer "F.Cu") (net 30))
 (segment (start 172.45 113.4) (end 168.7 109.65) (width 0.5) (layer "F.Cu") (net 30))
 (segment (start 169.205 106.445) (end 170.3 106.445) (width 0.5) (layer "F.Cu") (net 30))
 (segment (start 168.7 106.95) (end 169.205 106.445) (width 0.5) (layer "F.Cu") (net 30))
 (segment (start 179.5 113.4) (end 172.45 113.4) (width 0.5) (layer "F.Cu") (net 30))
 (via (at 179.5 113.4) (size 0.5) (drill 0.2) (layers "F.Cu" "B.Cu") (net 30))
 (segment (start 180.4 112.5) (end 179.5 113.4) (width 0.5) (layer "B.Cu") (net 30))
 (segment (start 182.65 112.5) (end 180.4 112.5) (width 0.5) (layer "B.Cu") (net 30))
 (segment (start 160.55 115.8) (end 179.2 115.8) (width 0.5) (layer "B.Cu") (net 13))
 (segment (start 180.5 114.5) (end 182.6 114.5) (width 0.5) (layer "B.Cu") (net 13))
 (segment (start 143.75 99) (end 160.55 115.8) (width 0.5) (layer "B.Cu") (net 13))
 (segment (start 179.2 115.8) (end 180.5 114.5) (width 0.5) (layer "B.Cu") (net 13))
 (segment (start 142.4 99) (end 143.75 99) (width 0.5) (layer "B.Cu") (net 13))
 (segment (start 144.55 101) (end 160.05 116.5) (width 0.5) (layer "B.Cu") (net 14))
 (segment (start 160.05 116.5) (end 182.5 116.5) (width 0.5) (layer "B.Cu") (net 14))
 (segment (start 142.3 101) (end 144.55 101) (width 0.5) (layer "B.Cu") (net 14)))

